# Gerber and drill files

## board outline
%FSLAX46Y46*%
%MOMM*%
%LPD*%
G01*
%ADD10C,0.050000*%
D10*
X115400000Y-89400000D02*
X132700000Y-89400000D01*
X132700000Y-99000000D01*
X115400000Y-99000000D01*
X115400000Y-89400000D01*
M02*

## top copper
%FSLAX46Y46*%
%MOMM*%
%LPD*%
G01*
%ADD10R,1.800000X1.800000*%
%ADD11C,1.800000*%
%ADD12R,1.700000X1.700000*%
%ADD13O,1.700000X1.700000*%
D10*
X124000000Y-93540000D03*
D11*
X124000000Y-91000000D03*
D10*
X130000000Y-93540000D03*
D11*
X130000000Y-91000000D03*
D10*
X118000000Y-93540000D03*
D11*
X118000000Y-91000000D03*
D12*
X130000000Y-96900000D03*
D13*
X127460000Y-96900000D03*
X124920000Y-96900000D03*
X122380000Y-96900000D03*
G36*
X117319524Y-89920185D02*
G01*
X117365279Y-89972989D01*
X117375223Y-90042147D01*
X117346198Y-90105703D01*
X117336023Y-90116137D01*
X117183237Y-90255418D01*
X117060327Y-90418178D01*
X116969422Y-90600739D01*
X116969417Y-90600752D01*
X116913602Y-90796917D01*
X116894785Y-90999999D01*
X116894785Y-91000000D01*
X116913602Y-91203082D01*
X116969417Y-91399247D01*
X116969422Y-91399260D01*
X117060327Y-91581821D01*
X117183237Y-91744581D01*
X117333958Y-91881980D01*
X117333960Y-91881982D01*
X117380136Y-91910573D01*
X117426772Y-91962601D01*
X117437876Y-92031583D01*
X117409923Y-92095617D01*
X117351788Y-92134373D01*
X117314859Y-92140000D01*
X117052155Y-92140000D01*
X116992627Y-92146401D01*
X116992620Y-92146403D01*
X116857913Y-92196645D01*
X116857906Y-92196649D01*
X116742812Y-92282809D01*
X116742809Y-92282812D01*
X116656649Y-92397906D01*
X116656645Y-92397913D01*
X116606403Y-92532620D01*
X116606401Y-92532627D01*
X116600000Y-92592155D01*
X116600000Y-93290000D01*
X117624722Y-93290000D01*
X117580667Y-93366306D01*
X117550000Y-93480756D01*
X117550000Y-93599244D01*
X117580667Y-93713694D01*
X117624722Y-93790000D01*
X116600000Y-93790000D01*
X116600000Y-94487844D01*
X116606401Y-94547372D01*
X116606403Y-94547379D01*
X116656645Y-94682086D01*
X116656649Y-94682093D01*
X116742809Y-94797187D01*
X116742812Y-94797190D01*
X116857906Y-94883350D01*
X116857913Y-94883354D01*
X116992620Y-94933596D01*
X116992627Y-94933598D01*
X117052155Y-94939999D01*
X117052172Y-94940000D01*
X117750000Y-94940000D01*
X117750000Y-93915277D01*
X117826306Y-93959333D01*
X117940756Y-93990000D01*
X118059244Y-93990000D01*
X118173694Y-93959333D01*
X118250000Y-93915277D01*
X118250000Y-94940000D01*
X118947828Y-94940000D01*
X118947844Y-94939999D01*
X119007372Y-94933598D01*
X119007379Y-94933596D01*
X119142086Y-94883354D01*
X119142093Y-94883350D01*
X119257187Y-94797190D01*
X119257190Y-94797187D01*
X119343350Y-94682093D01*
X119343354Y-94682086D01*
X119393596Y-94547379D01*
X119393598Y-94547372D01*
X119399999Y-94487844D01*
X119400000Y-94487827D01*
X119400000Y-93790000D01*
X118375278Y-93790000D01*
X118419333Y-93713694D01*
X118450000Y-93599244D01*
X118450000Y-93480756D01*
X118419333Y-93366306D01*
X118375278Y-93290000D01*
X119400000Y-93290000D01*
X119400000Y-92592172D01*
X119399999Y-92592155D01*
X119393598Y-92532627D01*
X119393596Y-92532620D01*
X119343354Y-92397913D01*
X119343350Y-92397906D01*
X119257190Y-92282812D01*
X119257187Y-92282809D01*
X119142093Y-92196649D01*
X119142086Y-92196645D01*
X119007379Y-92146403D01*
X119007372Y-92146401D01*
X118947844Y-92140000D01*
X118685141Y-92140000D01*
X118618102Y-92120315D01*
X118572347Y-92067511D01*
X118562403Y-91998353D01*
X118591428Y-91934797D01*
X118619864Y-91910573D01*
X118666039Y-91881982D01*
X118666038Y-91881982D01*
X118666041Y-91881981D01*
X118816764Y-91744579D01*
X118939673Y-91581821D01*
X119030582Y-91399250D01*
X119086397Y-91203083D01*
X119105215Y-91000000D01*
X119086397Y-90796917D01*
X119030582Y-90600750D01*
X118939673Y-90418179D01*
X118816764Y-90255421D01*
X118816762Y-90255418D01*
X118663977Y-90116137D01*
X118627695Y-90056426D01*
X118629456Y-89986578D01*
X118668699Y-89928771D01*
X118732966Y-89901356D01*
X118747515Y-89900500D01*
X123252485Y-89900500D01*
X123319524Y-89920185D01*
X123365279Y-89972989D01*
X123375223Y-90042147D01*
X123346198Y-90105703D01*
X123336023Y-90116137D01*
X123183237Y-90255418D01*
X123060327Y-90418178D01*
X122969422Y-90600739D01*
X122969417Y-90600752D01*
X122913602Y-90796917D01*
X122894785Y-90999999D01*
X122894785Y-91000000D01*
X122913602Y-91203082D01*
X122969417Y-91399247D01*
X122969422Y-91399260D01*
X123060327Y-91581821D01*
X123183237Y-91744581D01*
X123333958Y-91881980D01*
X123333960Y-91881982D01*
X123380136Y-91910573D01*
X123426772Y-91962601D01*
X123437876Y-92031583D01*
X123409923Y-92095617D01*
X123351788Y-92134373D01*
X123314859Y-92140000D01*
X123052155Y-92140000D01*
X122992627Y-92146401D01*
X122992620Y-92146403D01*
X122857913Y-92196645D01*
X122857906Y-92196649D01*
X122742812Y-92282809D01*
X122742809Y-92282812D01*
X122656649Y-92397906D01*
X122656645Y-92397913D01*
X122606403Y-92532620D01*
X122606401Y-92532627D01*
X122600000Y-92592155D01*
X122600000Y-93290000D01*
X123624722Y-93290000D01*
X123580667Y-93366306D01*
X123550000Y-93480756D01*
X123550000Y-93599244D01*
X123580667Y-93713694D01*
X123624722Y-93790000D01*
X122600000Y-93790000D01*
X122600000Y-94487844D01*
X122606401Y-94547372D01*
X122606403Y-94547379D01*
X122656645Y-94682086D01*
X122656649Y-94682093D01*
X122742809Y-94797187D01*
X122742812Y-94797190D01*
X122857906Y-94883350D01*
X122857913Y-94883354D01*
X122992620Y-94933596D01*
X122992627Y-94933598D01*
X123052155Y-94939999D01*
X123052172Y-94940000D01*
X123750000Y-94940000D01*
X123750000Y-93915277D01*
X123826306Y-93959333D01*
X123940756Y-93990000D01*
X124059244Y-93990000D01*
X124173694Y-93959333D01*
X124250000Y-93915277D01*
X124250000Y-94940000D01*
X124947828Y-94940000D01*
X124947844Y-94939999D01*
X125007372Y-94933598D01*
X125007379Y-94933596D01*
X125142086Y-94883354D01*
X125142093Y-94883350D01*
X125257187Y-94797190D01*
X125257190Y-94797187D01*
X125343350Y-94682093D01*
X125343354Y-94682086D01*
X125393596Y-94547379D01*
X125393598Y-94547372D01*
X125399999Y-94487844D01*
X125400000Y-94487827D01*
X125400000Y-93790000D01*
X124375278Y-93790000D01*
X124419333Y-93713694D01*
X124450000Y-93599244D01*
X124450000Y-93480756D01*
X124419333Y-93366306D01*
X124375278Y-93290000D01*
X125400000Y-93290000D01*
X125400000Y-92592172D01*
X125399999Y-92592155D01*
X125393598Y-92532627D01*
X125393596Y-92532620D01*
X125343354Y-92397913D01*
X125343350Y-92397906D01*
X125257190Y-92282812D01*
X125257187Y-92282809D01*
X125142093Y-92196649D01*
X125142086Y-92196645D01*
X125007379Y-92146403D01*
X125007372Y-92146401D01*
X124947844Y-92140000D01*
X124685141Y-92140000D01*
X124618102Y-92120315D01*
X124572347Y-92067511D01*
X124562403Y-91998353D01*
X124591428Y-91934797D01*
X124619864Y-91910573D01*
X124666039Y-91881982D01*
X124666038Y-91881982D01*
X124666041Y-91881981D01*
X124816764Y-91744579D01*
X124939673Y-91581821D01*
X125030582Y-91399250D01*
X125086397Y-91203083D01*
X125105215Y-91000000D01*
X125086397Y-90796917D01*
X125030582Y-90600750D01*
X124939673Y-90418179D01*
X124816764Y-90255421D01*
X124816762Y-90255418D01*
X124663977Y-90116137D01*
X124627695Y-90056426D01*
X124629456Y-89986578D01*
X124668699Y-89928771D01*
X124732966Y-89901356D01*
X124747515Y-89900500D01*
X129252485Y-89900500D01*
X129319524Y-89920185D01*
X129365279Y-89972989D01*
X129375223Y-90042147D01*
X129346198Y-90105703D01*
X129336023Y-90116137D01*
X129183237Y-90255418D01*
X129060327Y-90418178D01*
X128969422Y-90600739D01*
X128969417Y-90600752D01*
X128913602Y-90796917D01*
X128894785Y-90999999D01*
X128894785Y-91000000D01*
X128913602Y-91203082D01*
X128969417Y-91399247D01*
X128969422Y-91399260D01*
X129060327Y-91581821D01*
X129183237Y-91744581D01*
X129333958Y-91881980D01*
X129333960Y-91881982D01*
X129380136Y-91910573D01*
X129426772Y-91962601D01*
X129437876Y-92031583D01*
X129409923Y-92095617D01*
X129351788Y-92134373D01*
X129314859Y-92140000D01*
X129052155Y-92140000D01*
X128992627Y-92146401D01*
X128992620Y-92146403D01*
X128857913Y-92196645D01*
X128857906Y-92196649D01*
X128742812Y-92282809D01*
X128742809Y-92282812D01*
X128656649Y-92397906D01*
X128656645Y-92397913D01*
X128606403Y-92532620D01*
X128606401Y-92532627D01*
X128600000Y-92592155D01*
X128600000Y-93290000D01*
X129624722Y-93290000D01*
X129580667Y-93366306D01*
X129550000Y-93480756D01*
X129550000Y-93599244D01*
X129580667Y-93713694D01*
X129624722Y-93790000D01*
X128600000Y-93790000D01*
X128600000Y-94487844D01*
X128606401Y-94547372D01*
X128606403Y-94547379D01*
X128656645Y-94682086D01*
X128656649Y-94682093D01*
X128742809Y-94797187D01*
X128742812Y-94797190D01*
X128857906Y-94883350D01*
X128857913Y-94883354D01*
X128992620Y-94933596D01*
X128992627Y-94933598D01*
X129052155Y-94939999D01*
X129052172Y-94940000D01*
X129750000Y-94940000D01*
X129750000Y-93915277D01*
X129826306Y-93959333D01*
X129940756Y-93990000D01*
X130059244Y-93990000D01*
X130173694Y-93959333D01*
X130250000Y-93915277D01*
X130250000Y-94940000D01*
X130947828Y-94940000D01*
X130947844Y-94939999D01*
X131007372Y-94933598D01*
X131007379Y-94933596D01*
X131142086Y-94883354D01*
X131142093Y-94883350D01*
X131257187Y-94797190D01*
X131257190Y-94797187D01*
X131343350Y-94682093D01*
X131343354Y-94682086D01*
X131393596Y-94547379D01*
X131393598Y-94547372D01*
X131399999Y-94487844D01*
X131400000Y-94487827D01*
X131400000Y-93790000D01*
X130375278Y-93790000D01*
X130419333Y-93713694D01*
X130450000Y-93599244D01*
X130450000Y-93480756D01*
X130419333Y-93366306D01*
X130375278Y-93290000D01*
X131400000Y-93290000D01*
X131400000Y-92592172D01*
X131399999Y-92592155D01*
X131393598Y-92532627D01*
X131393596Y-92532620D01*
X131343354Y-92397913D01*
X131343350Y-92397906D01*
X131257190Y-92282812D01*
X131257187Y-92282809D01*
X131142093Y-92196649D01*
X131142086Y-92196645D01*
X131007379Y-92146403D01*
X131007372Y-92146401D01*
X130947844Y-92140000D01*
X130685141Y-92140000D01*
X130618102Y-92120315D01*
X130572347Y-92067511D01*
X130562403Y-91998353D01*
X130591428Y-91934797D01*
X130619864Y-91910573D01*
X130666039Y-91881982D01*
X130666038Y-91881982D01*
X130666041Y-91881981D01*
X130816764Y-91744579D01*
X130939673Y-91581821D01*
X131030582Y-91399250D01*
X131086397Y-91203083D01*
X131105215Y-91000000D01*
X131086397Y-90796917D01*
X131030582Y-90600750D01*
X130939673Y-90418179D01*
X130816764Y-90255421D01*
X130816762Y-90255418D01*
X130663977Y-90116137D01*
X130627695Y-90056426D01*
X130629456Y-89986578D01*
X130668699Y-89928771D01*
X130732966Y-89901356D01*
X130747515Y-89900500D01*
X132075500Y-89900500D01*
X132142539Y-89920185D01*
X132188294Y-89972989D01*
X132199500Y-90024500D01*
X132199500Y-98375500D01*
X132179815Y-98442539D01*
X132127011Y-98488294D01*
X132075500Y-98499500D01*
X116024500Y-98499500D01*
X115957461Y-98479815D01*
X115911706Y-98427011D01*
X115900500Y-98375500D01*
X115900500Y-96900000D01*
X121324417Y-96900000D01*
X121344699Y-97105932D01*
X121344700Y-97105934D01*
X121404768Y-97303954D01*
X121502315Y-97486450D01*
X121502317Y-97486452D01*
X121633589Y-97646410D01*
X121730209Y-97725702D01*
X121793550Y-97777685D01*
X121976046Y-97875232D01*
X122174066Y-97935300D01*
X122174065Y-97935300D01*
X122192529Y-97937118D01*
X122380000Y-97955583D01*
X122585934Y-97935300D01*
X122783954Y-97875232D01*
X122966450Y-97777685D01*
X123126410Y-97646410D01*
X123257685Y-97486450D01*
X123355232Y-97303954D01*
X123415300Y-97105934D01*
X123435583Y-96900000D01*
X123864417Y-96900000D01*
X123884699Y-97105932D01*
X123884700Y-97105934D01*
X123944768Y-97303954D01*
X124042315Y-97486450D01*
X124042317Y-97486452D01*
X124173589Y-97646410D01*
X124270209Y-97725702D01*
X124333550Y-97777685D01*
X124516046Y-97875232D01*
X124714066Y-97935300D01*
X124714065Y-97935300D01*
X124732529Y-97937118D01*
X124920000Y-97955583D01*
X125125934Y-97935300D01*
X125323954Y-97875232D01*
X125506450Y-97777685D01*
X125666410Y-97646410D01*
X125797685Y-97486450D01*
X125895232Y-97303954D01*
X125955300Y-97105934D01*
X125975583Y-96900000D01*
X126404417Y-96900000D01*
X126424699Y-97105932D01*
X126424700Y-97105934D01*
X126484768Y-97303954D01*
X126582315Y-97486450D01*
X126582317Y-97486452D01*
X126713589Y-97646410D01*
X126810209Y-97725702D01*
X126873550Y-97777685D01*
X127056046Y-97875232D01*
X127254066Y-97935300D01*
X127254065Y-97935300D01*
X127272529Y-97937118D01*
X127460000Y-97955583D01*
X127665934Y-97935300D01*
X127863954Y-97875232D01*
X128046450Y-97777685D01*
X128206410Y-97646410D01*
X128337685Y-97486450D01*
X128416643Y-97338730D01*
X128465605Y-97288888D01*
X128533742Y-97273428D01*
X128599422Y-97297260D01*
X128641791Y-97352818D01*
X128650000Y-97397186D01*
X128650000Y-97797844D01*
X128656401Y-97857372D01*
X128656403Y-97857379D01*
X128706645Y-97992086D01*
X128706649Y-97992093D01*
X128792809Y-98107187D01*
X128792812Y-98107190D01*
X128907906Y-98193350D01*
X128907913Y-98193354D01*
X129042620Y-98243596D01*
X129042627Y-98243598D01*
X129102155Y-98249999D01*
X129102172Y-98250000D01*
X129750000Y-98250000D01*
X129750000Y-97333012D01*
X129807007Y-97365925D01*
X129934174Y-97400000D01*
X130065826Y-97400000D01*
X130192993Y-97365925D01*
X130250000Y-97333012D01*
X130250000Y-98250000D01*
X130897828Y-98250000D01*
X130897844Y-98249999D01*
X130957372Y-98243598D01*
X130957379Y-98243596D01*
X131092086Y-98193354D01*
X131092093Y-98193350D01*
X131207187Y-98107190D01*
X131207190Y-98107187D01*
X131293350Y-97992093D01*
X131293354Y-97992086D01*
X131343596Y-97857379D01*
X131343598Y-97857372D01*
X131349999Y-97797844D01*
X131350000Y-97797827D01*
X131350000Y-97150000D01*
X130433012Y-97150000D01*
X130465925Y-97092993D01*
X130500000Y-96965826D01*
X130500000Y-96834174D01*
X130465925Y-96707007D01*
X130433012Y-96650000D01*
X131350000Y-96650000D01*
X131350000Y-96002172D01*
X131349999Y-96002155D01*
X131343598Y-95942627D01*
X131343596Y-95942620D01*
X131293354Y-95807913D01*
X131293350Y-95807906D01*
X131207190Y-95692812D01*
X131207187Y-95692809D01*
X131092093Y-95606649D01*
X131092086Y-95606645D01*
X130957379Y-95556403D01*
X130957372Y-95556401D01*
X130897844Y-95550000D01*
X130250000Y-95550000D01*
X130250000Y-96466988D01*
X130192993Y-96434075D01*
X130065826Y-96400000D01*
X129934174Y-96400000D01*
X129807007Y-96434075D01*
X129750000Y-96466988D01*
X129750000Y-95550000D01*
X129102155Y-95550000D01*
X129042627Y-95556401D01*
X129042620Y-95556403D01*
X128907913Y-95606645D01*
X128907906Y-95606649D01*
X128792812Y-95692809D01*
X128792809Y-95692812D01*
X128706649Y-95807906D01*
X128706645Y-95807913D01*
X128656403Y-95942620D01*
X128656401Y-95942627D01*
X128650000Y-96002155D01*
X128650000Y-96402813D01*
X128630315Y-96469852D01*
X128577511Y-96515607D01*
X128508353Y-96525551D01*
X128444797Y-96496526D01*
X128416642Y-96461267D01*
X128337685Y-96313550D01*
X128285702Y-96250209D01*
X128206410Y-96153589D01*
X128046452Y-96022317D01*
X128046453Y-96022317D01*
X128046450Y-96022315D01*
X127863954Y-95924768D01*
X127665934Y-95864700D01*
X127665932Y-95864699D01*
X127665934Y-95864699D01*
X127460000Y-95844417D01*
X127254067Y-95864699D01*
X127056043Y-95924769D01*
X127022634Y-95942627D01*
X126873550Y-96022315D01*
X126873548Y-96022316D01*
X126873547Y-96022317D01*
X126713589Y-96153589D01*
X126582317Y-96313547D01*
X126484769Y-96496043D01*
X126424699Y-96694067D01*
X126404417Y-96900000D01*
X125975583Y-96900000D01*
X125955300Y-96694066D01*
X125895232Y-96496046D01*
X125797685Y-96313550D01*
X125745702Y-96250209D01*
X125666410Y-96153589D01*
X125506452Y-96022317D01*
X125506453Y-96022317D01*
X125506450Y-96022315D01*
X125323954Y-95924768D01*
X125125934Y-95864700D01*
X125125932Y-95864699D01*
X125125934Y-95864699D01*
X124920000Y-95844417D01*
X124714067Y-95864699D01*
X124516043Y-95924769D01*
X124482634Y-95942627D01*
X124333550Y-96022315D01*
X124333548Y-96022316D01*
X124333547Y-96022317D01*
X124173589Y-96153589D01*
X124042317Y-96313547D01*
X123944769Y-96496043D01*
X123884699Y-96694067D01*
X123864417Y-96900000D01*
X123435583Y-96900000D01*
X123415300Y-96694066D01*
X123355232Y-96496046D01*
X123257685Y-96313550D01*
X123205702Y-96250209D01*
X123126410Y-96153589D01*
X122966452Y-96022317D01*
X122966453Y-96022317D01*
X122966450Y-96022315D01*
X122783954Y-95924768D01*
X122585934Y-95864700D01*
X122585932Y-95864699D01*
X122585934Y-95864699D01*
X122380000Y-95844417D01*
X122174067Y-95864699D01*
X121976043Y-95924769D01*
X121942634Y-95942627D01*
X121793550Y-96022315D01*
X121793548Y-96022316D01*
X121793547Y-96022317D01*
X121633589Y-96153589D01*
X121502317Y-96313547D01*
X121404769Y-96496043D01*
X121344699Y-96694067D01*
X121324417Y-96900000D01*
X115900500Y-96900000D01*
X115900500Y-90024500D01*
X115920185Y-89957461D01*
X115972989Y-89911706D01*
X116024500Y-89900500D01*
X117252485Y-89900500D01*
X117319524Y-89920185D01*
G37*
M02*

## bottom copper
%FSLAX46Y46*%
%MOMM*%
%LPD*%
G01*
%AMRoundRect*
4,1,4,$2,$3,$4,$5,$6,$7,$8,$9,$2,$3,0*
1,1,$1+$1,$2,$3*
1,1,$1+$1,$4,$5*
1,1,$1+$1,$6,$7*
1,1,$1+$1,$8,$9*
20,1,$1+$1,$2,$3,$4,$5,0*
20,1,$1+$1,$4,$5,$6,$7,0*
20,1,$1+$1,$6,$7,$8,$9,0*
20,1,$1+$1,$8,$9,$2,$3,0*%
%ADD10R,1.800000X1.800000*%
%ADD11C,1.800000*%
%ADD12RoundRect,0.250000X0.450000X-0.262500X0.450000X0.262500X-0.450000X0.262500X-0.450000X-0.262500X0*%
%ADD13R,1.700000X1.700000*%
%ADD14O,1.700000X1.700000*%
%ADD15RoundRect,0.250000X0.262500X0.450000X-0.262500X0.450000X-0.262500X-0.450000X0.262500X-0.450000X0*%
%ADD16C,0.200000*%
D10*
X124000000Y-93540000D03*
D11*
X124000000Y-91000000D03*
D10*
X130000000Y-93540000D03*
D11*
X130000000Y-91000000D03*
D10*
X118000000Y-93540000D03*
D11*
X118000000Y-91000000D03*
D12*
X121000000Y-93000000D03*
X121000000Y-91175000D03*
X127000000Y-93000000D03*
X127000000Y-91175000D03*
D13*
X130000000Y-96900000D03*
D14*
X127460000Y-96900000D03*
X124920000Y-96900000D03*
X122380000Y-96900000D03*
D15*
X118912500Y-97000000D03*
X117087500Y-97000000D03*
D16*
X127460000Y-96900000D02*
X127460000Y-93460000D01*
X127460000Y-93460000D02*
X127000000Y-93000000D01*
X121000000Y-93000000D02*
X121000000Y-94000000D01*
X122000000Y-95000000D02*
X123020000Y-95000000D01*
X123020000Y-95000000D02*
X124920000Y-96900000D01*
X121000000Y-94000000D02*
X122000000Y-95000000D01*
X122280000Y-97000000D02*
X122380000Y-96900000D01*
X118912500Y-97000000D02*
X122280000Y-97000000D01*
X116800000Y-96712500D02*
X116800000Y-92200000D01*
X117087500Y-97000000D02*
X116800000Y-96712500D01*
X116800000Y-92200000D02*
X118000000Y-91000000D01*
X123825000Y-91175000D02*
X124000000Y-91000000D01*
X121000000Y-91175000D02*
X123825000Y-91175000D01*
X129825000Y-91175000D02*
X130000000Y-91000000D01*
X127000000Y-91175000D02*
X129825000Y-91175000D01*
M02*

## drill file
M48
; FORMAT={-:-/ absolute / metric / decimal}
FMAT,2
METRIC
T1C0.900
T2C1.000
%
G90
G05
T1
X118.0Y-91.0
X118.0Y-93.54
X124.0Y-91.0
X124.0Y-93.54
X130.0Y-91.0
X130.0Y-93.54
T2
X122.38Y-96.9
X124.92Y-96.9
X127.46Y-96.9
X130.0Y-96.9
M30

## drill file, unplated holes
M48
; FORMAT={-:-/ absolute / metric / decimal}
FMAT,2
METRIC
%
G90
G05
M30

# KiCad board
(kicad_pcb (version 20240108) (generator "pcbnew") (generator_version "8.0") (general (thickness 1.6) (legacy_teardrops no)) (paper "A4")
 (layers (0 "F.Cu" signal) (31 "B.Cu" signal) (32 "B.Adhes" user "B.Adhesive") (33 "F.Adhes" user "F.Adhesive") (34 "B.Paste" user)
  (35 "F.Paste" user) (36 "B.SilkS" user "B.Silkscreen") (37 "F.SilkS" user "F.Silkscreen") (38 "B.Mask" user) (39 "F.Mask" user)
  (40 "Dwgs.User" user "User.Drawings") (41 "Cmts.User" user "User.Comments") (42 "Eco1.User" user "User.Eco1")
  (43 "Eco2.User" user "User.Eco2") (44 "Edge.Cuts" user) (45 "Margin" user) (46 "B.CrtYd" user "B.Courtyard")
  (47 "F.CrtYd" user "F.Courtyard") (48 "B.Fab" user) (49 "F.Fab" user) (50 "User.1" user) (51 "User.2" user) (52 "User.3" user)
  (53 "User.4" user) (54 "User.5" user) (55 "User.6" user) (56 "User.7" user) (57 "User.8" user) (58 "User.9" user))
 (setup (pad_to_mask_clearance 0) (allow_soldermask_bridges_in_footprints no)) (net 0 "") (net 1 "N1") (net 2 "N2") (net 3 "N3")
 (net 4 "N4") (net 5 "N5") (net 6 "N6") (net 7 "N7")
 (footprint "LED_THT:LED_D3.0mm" (layer "F.Cu") (at 124 93.54 90)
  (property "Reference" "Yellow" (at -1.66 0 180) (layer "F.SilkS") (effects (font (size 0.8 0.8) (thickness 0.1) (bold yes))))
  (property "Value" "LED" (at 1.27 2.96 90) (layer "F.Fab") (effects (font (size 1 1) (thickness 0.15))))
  (pad "1" thru_hole rect (at 0 0 90) (size 1.8 1.8) (drill 0.9) (layers "*.Cu" "*.Mask") (remove_unused_layers no) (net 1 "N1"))
  (pad "2" thru_hole circle (at 2.54 0 90) (size 1.8 1.8) (drill 0.9) (layers "*.Cu" "*.Mask") (remove_unused_layers no) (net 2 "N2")))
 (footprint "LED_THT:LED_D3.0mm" (layer "F.Cu") (at 130 93.54 90)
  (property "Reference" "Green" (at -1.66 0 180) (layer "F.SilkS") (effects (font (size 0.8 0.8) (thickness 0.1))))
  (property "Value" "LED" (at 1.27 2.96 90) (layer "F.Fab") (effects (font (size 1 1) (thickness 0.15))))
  (pad "1" thru_hole rect (at 0 0 90) (size 1.8 1.8) (drill 0.9) (layers "*.Cu" "*.Mask") (remove_unused_layers no) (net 1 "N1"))
  (pad "2" thru_hole circle (at 2.54 0 90) (size 1.8 1.8) (drill 0.9) (layers "*.Cu" "*.Mask") (remove_unused_layers no) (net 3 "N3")))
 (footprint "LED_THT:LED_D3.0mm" (layer "F.Cu") (at 118 93.54 90)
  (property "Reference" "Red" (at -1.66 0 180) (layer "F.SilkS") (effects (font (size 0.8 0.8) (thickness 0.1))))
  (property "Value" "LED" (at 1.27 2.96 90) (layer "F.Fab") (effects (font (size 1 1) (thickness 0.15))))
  (pad "1" thru_hole rect (at 0 0 90) (size 1.8 1.8) (drill 0.9) (layers "*.Cu" "*.Mask") (remove_unused_layers no) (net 1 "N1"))
  (pad "2" thru_hole circle (at 2.54 0 90) (size 1.8 1.8) (drill 0.9) (layers "*.Cu" "*.Mask") (remove_unused_layers no) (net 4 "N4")))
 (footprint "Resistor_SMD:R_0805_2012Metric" (layer "B.Cu") (at 121 92.0875 90)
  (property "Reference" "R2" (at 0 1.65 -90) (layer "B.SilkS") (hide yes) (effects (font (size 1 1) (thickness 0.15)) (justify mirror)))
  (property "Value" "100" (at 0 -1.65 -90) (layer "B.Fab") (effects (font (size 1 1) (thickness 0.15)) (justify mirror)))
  (pad "1" smd roundrect (at -0.9125 0 90) (size 1.025 1.4) (layers "B.Cu" "B.Paste" "B.Mask") (roundrect_rratio 0.243902) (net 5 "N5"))
  (pad "2" smd roundrect (at 0.9125 0 90) (size 1.025 1.4) (layers "B.Cu" "B.Paste" "B.Mask") (roundrect_rratio 0.243902) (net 2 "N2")))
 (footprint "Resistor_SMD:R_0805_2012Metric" (layer "B.Cu") (at 127 92.0875 90)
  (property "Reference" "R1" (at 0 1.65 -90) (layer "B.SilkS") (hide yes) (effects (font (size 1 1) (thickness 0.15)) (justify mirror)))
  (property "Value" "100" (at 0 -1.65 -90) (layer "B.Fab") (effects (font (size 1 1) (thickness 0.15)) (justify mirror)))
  (pad "1" smd roundrect (at -0.9125 0 90) (size 1.025 1.4) (layers "B.Cu" "B.Paste" "B.Mask") (roundrect_rratio 0.243902) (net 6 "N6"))
  (pad "2" smd roundrect (at 0.9125 0 90) (size 1.025 1.4) (layers "B.Cu" "B.Paste" "B.Mask") (roundrect_rratio 0.243902) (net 3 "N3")))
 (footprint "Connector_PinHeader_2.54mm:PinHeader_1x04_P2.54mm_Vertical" (layer "B.Cu") (at 130 96.9 90)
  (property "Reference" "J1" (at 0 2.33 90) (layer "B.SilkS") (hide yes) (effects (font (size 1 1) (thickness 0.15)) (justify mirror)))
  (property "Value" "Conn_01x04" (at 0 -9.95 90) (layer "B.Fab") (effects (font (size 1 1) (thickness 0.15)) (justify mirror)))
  (pad "1" thru_hole rect (at 0 0 90) (size 1.7 1.7) (drill 1) (layers "*.Cu" "*.Mask") (remove_unused_layers no) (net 1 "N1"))
  (pad "2" thru_hole oval (at 0 -2.54 90) (size 1.7 1.7) (drill 1) (layers "*.Cu" "*.Mask") (remove_unused_layers no) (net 6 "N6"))
  (pad "3" thru_hole oval (at 0 -5.08 90) (size 1.7 1.7) (drill 1) (layers "*.Cu" "*.Mask") (remove_unused_layers no) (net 5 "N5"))
  (pad "4" thru_hole oval (at 0 -7.62 90) (size 1.7 1.7) (drill 1) (layers "*.Cu" "*.Mask") (remove_unused_layers no) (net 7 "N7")))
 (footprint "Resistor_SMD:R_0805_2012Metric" (layer "B.Cu") (at 118 97 180)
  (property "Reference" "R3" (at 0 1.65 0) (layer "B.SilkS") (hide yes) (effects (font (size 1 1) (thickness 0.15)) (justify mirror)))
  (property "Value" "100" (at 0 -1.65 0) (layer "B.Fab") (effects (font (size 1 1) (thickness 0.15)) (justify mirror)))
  (pad "1" smd roundrect (at -0.9125 0 180) (size 1.025 1.4) (layers "B.Cu" "B.Paste" "B.Mask") (roundrect_rratio 0.243902) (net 7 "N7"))
  (pad "2" smd roundrect (at 0.9125 0 180) (size 1.025 1.4) (layers "B.Cu" "B.Paste" "B.Mask") (roundrect_rratio 0.243902) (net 4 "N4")))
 (gr_rect (start 115.4 89.4) (end 132.7 99) (stroke (width 0.05) (type default)) (fill none) (layer "Edge.Cuts"))
 (segment (start 127.46 96.9) (end 127.46 93.46) (width 0.2) (layer "B.Cu") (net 6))
 (segment (start 127.46 93.46) (end 127 93) (width 0.2) (layer "B.Cu") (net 6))
 (segment (start 121 93) (end 121 94) (width 0.2) (layer "B.Cu") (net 5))
 (segment (start 122 95) (end 123.02 95) (width 0.2) (layer "B.Cu") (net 5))
 (segment (start 123.02 95) (end 124.92 96.9) (width 0.2) (layer "B.Cu") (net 5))
 (segment (start 121 94) (end 122 95) (width 0.2) (layer "B.Cu") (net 5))
 (segment (start 122.28 97) (end 122.38 96.9) (width 0.2) (layer "B.Cu") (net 7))
 (segment (start 118.9125 97) (end 122.28 97) (width 0.2) (layer "B.Cu") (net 7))
 (segment (start 116.8 96.7125) (end 116.8 92.2) (width 0.2) (layer "B.Cu") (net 4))
 (segment (start 117.0875 97) (end 116.8 96.7125) (width 0.2) (layer "B.Cu") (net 4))
 (segment (start 116.8 92.2) (end 118 91) (width 0.2) (layer "B.Cu") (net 4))
 (segment (start 123.825 91.175) (end 124 91) (width 0.2) (layer "B.Cu") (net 2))
 (segment (start 121 91.175) (end 123.825 91.175) (width 0.2) (layer "B.Cu") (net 2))
 (segment (start 129.825 91.175) (end 130 91) (width 0.2) (layer "B.Cu") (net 3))
 (segment (start 127 91.175) (end 129.825 91.175) (width 0.2) (layer "B.Cu") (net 3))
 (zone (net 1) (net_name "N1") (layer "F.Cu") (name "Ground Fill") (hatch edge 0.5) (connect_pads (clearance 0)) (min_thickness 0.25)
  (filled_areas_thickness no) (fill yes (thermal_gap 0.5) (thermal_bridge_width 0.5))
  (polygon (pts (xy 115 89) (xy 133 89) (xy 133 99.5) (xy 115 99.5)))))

